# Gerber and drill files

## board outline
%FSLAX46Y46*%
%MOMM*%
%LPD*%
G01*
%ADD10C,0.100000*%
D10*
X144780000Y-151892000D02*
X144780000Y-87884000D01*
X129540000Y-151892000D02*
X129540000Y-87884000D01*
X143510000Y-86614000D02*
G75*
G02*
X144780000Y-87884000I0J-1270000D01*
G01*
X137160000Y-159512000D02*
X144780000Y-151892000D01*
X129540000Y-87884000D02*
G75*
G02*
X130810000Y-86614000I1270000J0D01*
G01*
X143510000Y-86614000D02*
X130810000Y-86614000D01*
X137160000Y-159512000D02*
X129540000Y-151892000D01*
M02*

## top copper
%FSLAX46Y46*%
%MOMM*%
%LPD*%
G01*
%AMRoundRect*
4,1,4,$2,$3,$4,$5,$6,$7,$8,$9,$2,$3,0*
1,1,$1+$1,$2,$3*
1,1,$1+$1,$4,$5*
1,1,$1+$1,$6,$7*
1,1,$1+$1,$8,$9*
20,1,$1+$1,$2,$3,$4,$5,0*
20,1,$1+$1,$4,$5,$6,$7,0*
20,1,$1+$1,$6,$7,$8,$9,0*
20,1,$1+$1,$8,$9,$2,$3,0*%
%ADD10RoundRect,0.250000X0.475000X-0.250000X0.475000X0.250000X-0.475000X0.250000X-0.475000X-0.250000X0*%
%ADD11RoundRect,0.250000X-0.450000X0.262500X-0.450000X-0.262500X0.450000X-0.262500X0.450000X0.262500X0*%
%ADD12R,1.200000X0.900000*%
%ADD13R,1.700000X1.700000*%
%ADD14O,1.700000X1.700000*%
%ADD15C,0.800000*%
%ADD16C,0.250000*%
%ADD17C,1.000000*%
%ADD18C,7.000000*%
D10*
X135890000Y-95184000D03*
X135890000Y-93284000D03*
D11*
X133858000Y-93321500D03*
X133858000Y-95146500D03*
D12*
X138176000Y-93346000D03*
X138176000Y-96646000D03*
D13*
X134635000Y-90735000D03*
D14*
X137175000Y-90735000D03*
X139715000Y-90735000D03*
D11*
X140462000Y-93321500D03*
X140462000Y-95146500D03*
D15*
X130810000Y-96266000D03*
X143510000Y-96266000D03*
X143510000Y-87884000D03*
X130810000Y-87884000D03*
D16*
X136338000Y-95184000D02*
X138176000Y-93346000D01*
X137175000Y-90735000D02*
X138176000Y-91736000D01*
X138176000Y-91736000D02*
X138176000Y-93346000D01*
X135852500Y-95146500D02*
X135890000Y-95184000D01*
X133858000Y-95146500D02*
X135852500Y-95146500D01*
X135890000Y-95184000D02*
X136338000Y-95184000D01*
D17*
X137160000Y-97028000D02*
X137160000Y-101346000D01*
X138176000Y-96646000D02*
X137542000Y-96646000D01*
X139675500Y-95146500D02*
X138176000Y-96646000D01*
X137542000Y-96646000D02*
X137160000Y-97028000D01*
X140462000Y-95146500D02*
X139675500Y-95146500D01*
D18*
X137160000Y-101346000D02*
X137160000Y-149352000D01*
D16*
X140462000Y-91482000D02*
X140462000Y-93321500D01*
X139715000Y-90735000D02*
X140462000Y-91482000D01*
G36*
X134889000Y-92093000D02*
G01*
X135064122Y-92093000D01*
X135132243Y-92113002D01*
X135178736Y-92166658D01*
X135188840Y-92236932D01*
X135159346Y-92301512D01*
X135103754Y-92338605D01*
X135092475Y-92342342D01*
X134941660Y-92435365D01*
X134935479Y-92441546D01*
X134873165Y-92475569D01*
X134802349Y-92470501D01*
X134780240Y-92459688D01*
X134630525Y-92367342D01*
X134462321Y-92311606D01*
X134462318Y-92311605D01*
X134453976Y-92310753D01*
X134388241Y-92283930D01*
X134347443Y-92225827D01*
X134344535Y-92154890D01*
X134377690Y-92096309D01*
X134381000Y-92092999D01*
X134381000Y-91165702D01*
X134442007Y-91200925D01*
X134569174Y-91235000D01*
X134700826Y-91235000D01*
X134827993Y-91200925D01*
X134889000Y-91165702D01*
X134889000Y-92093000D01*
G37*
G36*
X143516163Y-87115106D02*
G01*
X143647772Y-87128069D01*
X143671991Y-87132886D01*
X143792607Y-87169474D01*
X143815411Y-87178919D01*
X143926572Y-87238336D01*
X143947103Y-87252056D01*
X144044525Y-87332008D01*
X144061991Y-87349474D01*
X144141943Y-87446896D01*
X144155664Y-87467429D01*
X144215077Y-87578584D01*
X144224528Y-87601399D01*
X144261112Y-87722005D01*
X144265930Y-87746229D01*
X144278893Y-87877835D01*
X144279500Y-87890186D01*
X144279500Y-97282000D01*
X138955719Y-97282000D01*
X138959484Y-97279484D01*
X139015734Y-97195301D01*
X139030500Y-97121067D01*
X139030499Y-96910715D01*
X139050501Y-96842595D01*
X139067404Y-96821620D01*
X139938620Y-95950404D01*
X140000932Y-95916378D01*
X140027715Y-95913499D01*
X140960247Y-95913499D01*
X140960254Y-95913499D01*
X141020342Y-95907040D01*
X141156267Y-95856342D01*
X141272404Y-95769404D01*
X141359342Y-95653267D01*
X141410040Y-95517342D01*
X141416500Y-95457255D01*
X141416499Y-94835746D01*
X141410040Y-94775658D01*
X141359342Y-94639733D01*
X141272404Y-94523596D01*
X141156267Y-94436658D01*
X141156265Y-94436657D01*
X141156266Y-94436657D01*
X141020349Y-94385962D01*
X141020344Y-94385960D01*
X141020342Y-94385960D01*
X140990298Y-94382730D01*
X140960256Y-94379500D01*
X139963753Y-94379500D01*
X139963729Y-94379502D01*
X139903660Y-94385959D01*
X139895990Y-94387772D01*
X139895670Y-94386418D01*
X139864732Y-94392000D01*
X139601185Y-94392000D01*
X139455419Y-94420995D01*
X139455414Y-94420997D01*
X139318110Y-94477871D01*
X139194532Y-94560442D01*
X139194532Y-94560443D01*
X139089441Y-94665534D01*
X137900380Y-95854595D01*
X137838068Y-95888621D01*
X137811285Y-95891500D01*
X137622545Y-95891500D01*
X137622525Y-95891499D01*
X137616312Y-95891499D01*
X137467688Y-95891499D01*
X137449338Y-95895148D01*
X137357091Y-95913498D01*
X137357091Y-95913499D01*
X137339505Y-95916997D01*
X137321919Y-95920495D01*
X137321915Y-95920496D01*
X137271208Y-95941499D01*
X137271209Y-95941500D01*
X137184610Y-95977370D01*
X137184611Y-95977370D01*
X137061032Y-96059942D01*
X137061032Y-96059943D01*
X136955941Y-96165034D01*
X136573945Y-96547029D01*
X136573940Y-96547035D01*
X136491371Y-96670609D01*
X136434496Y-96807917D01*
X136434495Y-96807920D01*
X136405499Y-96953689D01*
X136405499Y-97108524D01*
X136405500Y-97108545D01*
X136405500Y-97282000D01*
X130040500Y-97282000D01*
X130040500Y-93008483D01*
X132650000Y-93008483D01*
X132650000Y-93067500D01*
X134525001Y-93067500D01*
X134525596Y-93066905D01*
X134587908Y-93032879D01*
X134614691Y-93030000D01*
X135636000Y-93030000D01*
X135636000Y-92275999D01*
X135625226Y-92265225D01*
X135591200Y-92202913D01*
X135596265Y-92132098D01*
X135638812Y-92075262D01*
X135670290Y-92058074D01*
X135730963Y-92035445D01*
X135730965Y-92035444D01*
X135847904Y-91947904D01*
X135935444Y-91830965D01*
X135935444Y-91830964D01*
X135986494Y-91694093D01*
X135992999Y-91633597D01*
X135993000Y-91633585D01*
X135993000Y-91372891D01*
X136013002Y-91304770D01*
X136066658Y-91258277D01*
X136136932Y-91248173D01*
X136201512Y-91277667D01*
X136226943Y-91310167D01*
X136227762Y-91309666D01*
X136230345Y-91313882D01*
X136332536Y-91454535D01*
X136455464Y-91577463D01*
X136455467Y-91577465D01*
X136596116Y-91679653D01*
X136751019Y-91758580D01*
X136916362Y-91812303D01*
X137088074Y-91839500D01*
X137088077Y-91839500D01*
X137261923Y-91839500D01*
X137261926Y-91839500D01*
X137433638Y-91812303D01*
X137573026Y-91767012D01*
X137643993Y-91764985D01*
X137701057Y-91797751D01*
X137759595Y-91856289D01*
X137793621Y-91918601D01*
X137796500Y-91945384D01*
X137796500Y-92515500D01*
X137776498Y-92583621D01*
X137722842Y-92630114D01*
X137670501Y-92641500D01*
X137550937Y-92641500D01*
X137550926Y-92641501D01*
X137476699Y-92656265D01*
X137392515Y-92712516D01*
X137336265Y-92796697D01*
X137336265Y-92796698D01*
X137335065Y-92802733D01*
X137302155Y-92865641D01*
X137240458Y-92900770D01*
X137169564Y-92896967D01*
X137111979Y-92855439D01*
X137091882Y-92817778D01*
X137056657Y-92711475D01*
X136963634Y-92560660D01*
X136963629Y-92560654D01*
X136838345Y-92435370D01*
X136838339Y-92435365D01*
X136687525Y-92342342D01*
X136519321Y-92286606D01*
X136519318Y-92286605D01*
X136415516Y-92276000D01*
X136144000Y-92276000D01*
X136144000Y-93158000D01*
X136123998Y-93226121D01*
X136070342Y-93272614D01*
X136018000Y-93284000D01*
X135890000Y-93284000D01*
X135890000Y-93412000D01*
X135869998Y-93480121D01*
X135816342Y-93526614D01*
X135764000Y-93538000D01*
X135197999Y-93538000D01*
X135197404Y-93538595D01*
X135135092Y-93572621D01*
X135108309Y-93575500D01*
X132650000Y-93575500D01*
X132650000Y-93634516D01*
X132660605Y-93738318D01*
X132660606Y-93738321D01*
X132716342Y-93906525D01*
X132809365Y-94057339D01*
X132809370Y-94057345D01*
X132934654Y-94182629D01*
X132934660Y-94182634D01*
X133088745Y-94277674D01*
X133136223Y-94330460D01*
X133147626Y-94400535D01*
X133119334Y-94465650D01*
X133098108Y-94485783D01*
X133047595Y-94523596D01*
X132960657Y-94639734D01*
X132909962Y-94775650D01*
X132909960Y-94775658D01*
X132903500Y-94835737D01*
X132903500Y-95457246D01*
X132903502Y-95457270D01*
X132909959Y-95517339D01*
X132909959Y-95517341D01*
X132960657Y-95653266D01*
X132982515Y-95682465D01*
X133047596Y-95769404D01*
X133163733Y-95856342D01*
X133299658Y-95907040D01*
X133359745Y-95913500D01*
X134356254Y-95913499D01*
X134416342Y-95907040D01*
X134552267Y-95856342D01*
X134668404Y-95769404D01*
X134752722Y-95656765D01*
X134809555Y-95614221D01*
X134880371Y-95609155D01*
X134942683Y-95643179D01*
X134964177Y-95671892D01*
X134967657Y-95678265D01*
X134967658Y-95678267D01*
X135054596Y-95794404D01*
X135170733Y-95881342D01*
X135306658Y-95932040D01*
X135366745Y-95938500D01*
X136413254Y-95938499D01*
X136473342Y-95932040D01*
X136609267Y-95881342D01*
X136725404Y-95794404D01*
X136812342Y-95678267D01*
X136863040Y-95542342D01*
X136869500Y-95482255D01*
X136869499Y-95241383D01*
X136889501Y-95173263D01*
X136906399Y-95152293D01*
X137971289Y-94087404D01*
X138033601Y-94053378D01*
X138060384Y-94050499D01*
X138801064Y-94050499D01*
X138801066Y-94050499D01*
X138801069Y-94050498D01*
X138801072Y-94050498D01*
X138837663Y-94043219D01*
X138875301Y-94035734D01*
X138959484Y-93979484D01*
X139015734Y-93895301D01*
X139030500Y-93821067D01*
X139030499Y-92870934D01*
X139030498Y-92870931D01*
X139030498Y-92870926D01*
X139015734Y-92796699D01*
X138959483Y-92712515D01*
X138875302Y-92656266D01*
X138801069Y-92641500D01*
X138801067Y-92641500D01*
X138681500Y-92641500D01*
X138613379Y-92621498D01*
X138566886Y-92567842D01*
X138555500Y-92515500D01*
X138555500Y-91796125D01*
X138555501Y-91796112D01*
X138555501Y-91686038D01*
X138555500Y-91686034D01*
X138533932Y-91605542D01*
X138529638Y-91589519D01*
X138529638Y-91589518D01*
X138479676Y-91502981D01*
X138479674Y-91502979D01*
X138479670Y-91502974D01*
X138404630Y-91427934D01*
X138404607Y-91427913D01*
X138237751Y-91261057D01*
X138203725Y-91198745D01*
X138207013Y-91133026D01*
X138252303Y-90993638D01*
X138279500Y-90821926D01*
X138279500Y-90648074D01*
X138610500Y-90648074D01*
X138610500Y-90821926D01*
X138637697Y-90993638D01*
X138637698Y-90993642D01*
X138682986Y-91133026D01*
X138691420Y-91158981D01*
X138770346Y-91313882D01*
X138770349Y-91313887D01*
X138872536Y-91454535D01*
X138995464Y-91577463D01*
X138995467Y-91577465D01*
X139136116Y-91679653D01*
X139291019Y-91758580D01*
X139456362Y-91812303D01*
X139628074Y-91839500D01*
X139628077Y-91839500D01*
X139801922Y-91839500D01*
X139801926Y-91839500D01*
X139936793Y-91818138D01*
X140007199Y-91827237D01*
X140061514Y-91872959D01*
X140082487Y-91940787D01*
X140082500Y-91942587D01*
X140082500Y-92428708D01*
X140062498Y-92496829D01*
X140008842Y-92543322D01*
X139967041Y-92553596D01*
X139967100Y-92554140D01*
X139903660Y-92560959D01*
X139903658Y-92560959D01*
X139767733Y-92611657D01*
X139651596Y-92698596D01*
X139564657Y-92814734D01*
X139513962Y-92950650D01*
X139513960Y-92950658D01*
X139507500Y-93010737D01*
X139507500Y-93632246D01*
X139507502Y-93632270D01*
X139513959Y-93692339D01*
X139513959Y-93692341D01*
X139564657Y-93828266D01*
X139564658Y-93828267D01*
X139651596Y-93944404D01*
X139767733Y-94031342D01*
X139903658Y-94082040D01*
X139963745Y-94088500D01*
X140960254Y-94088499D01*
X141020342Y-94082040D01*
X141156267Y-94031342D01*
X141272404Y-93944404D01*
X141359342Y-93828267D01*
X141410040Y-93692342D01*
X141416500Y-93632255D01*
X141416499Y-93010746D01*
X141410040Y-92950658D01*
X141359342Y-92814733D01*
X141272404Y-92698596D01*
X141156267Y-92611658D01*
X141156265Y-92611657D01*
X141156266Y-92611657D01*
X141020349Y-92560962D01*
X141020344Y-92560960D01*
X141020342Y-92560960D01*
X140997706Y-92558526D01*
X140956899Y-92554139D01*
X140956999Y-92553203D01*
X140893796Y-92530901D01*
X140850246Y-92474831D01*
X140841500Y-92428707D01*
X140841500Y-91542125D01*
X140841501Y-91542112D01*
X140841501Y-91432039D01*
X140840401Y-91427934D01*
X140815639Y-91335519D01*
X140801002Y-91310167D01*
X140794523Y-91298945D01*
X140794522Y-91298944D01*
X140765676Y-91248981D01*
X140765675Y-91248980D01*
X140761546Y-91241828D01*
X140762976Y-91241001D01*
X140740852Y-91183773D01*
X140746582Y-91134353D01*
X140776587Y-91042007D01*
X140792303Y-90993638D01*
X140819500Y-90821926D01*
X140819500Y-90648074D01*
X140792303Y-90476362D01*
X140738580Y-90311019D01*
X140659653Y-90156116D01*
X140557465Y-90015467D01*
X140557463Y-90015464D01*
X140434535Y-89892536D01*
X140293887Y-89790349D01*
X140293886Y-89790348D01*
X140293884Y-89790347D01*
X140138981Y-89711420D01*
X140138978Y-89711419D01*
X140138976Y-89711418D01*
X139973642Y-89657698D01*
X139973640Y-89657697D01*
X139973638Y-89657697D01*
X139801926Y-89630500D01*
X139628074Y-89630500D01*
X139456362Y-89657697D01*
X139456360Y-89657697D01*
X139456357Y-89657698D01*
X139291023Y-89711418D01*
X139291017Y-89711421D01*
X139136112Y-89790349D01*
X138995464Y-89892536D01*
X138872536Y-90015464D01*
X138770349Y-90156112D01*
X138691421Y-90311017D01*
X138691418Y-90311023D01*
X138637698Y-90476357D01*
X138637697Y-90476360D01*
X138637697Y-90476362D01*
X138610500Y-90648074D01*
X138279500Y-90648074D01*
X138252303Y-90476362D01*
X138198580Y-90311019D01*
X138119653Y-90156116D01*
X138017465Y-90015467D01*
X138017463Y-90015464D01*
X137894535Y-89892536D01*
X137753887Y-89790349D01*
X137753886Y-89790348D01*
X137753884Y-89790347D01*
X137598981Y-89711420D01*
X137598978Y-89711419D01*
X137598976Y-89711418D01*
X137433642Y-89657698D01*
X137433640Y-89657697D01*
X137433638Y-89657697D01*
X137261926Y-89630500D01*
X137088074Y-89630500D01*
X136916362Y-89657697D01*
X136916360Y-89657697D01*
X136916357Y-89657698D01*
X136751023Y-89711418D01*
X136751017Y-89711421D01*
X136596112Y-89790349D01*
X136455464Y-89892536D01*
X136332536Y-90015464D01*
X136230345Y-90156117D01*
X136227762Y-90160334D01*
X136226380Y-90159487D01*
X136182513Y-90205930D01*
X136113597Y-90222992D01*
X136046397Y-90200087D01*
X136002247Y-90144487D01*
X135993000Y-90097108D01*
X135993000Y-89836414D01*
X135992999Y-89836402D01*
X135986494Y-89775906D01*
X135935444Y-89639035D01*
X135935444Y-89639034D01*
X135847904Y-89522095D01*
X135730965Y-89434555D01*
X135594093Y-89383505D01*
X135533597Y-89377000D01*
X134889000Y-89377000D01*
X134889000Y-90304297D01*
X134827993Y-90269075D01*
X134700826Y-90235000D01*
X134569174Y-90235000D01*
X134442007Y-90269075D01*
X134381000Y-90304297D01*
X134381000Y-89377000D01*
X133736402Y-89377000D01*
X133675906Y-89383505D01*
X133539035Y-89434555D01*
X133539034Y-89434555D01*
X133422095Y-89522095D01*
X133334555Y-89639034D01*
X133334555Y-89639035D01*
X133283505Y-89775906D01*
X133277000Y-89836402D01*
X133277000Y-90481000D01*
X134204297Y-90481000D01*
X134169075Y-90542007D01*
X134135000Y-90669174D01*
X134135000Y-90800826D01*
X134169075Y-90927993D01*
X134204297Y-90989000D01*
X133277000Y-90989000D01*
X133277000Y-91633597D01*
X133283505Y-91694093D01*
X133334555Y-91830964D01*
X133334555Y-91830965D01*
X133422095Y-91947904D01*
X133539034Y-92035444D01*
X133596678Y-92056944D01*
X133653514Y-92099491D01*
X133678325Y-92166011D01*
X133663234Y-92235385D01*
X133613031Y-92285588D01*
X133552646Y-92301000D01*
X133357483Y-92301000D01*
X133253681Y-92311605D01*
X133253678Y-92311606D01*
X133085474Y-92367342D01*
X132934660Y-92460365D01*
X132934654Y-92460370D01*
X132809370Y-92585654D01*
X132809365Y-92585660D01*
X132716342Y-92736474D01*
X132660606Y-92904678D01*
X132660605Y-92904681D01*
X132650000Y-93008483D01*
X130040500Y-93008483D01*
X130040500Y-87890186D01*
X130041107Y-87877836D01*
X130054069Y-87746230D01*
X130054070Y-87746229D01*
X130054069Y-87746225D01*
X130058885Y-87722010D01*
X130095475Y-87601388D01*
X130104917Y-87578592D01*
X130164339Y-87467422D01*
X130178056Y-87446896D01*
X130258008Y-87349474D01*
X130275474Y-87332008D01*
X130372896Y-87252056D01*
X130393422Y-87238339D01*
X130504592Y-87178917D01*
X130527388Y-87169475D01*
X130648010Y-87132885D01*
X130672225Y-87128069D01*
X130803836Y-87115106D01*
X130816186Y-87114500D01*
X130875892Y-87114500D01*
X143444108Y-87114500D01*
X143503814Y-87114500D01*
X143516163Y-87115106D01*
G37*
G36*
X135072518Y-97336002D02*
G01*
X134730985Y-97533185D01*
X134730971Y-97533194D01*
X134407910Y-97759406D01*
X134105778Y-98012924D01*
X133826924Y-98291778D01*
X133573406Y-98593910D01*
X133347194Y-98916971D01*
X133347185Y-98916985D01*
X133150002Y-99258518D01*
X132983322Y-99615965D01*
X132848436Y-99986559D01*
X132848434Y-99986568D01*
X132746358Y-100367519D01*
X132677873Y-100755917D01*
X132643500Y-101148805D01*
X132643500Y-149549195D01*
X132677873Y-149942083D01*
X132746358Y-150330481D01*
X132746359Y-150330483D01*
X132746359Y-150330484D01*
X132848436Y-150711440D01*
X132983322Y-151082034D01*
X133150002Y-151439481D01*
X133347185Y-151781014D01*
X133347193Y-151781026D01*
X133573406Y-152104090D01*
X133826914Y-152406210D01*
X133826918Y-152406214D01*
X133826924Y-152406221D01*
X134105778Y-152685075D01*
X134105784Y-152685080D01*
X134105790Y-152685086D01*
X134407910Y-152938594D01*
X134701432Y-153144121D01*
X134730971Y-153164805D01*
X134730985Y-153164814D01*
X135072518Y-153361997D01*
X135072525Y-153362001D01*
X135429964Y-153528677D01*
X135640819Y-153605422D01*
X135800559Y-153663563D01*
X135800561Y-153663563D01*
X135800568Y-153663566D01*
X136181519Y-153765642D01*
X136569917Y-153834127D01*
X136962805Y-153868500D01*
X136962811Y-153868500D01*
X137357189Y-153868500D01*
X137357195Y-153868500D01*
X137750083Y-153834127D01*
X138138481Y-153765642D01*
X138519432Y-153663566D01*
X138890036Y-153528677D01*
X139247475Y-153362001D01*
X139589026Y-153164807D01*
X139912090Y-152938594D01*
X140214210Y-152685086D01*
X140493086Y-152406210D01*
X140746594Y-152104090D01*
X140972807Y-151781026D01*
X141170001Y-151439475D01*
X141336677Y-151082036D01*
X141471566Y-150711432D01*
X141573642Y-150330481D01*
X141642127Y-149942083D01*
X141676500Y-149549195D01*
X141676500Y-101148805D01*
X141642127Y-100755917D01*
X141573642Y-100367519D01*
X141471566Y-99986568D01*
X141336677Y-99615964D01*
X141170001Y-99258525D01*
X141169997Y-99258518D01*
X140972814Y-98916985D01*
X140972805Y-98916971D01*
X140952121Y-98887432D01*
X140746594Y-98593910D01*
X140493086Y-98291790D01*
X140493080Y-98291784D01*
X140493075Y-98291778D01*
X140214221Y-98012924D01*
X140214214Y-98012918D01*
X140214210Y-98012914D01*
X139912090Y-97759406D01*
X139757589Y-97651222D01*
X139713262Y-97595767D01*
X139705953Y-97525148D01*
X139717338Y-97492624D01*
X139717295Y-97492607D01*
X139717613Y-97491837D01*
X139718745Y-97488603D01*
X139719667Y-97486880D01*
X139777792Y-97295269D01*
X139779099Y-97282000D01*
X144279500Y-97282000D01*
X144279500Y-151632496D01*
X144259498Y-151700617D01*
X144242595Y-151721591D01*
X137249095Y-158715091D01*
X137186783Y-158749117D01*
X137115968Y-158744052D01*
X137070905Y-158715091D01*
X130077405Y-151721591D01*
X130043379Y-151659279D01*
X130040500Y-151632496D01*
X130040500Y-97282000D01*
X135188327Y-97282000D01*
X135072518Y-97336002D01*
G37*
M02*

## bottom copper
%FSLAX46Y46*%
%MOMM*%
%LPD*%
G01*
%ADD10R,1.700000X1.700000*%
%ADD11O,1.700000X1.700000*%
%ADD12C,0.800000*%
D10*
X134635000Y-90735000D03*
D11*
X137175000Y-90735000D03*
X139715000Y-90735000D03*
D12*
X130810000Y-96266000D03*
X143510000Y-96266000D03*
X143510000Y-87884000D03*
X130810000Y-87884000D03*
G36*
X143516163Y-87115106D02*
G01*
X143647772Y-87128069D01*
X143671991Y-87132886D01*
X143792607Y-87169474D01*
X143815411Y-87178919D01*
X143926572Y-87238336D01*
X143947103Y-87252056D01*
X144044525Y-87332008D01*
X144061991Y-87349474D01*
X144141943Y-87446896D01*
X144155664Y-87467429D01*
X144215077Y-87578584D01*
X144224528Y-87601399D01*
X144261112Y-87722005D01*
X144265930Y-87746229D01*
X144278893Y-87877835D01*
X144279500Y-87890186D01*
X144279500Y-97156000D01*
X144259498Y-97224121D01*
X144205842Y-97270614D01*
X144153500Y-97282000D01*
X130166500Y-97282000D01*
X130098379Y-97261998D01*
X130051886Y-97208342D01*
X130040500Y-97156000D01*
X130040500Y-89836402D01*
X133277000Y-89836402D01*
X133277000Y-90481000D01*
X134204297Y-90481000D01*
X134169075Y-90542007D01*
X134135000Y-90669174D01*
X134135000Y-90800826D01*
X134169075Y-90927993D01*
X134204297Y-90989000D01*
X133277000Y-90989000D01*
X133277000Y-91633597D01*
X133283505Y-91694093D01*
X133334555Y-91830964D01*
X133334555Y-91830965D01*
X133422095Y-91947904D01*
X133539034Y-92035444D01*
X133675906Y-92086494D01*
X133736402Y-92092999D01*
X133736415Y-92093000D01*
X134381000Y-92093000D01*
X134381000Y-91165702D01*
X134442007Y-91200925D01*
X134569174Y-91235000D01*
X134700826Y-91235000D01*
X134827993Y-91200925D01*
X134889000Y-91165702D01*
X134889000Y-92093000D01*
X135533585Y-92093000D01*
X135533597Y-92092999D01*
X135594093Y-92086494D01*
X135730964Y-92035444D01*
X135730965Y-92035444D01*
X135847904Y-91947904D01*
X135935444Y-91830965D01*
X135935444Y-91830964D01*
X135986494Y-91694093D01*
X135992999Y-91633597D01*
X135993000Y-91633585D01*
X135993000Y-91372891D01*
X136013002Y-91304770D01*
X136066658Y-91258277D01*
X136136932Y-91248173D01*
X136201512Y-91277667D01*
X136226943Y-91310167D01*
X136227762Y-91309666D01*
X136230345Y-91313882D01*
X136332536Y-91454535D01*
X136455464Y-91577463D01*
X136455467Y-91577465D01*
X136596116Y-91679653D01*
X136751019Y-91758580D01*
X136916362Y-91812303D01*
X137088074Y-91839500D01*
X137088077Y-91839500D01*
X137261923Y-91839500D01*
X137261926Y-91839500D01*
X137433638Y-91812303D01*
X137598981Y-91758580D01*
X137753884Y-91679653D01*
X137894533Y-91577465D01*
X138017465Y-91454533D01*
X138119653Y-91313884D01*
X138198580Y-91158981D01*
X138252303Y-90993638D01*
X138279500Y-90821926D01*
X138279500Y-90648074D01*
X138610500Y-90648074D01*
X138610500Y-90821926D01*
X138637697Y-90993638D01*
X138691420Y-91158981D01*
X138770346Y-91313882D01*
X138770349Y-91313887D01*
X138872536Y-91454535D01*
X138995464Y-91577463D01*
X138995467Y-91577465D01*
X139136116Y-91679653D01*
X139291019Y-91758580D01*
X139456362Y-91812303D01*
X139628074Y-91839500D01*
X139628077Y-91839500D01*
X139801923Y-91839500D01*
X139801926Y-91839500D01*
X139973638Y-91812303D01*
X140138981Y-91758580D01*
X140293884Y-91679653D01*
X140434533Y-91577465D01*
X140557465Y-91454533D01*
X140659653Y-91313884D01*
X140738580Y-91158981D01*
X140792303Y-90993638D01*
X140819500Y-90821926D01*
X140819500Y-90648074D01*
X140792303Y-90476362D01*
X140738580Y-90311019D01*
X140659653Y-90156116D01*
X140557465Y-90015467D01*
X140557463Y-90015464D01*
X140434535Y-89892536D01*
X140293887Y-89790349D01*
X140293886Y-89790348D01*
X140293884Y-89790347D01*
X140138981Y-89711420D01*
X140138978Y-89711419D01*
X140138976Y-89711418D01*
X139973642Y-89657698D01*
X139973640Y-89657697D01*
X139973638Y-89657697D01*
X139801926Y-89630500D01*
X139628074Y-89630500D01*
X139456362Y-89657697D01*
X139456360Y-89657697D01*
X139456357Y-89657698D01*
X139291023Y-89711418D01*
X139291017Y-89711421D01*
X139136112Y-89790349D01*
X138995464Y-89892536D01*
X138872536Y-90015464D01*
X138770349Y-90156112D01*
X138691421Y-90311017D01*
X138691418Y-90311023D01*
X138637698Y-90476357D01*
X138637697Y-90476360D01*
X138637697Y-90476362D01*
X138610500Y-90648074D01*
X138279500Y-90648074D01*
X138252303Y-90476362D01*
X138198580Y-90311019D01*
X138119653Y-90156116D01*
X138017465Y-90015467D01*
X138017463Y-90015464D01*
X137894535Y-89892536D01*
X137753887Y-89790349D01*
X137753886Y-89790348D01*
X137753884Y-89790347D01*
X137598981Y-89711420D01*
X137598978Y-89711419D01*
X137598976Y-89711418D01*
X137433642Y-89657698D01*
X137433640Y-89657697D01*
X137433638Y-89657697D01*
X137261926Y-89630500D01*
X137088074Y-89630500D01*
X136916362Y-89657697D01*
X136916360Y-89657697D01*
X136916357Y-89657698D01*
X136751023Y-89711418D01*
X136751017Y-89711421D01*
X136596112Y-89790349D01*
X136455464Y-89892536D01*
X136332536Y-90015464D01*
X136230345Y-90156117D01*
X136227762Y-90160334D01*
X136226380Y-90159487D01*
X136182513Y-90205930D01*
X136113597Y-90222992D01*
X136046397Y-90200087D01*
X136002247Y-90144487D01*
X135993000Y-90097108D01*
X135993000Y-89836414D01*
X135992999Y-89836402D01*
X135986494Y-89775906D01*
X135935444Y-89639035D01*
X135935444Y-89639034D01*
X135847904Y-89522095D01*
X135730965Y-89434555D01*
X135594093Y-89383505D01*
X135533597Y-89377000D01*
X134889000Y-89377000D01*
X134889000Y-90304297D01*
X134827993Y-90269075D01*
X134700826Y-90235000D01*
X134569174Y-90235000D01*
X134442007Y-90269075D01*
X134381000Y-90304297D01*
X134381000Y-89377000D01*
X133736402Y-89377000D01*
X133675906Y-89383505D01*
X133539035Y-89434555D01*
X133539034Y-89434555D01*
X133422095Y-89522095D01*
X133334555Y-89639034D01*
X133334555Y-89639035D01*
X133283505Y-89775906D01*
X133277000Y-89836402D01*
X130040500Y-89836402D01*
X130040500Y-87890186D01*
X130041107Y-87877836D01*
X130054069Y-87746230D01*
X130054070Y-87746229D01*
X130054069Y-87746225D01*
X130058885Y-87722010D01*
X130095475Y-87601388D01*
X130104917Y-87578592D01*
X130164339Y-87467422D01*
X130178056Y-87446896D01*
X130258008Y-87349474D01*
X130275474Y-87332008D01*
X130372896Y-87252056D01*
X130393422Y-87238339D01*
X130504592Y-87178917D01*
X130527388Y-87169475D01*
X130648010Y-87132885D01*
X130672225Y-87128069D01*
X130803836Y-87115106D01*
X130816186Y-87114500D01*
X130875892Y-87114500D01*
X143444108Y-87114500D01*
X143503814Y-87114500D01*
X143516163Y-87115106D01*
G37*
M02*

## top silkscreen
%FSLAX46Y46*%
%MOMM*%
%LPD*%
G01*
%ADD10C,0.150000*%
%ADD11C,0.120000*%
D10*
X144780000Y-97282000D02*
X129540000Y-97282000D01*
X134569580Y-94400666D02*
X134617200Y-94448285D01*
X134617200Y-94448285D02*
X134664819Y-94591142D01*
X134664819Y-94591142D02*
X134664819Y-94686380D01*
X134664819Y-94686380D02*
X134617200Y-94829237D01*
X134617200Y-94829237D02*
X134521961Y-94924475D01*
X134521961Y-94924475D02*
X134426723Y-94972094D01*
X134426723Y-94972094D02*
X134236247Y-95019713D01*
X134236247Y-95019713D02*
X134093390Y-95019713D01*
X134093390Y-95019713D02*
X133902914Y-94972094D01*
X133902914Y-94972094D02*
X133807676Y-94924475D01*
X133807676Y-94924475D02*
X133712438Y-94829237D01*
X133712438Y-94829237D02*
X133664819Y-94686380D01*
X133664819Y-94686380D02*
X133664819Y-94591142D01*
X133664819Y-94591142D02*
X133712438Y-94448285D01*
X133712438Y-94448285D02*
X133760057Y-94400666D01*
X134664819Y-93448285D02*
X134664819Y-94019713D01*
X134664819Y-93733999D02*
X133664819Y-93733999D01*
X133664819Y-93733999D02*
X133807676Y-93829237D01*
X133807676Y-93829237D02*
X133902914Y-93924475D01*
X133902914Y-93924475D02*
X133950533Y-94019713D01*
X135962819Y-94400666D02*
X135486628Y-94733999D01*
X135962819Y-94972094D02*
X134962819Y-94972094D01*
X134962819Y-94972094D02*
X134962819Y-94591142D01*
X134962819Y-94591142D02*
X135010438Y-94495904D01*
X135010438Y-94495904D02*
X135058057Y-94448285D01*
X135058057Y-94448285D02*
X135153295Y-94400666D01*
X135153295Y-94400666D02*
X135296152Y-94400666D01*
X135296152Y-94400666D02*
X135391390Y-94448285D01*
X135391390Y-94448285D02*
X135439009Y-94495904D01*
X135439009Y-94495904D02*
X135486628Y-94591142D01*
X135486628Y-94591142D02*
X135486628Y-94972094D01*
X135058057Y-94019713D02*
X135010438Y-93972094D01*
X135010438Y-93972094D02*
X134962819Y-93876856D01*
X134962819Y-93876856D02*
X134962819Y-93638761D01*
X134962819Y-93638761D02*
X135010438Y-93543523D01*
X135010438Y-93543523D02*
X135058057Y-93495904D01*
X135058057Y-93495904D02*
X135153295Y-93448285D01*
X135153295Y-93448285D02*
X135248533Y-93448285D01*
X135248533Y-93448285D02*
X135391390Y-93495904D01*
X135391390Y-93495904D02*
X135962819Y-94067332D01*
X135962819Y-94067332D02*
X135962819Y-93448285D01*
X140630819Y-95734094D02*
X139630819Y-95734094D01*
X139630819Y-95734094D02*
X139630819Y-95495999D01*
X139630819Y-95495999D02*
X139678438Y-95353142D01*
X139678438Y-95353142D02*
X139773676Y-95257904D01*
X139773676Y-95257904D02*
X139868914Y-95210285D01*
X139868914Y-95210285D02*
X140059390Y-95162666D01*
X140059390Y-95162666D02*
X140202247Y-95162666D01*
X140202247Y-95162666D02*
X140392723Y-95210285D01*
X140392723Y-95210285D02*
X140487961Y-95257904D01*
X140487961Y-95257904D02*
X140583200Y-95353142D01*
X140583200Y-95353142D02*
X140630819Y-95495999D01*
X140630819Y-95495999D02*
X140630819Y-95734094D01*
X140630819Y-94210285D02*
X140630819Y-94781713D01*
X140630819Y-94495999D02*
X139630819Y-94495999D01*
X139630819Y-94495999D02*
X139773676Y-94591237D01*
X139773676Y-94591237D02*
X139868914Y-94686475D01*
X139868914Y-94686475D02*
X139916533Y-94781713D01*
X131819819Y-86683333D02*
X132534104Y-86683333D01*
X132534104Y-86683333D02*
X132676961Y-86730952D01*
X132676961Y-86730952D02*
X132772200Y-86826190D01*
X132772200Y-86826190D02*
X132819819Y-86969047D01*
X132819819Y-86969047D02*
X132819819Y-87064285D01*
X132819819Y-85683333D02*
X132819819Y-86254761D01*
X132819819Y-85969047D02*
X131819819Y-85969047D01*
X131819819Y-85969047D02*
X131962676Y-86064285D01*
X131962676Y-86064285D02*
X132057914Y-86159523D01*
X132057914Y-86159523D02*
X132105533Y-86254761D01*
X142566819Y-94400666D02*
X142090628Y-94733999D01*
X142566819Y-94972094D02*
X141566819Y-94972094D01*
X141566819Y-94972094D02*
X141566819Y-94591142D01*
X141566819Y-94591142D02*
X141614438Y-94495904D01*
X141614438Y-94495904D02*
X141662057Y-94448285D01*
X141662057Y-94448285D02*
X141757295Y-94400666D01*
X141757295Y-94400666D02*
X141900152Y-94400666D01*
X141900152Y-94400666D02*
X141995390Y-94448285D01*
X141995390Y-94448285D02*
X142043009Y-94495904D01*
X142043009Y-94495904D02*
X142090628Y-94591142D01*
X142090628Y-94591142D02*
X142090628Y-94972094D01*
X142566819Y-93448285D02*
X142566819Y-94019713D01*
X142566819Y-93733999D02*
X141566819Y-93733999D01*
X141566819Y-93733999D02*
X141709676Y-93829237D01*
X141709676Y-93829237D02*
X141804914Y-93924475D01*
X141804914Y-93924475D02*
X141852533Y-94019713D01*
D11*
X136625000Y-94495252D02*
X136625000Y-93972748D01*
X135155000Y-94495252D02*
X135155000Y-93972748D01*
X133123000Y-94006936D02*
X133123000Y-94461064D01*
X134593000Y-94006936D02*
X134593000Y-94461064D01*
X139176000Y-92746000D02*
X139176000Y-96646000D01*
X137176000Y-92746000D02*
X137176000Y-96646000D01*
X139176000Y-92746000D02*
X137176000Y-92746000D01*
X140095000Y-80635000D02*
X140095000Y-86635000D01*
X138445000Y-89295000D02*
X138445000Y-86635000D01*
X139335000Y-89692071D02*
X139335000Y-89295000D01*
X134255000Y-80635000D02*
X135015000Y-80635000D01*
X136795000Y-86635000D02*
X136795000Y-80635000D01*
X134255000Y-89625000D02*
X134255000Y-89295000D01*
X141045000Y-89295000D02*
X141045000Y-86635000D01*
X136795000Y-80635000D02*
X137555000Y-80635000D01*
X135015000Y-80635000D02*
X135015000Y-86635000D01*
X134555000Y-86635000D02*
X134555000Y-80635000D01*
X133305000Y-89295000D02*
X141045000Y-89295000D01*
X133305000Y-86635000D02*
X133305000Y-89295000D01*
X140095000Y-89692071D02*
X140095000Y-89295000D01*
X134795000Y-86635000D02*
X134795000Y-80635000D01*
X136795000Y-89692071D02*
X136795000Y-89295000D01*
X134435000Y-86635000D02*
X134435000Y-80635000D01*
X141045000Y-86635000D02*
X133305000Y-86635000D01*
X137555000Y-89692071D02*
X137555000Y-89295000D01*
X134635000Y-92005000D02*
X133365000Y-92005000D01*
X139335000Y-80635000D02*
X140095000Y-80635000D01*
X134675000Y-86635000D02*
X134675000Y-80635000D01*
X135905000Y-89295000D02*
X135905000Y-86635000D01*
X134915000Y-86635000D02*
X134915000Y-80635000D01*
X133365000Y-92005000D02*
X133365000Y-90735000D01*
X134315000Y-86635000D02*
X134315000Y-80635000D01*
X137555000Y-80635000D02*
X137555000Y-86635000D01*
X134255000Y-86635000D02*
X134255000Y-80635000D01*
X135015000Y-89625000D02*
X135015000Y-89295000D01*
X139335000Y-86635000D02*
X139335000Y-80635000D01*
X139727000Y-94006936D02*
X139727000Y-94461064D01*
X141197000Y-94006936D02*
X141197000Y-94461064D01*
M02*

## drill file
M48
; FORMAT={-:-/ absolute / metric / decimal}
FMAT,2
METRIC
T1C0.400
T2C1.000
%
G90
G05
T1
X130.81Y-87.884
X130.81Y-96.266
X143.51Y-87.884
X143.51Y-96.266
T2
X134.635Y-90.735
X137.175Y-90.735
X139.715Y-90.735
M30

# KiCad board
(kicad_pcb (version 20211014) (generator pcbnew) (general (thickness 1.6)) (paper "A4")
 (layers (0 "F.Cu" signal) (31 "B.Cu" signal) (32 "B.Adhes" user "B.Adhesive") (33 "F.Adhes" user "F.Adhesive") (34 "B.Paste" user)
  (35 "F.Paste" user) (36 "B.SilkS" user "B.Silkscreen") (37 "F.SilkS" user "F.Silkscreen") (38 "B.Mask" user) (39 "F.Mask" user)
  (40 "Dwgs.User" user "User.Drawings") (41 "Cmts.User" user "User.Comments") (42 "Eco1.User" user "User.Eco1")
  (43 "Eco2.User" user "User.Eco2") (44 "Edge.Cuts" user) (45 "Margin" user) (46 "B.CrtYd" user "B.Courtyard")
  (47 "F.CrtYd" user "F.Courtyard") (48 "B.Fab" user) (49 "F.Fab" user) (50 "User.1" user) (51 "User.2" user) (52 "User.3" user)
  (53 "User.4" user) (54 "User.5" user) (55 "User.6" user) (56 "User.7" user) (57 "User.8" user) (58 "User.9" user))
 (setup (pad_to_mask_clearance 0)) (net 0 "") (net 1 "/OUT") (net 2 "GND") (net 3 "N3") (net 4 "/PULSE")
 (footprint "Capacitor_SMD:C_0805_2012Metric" (layer "F.Cu") (at 135.89 94.234 90)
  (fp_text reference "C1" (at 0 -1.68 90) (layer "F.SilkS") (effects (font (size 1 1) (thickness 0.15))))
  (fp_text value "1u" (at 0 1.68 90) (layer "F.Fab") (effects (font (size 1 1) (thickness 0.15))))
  (fp_line (start -0.261252 0.735) (end 0.261252 0.735) (layer "F.SilkS") (width 0.12))
  (fp_line (start -0.261252 -0.735) (end 0.261252 -0.735) (layer "F.SilkS") (width 0.12))
  (pad "1" smd roundrect (at -0.95 0 90) (size 1 1.45) (layers "F.Cu" "F.Paste" "F.Mask") (roundrect_rratio 0.25) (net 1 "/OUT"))
  (pad "2" smd roundrect (at 0.95 0 90) (size 1 1.45) (layers "F.Cu" "F.Paste" "F.Mask") (roundrect_rratio 0.25) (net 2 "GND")))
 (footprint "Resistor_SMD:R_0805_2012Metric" (layer "F.Cu") (at 133.858 94.234 -90)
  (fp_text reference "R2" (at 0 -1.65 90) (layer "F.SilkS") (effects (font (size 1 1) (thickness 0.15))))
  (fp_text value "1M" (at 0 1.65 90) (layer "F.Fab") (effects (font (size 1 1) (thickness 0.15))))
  (fp_line (start -0.227064 0.735) (end 0.227064 0.735) (layer "F.SilkS") (width 0.12))
  (fp_line (start -0.227064 -0.735) (end 0.227064 -0.735) (layer "F.SilkS") (width 0.12))
  (pad "1" smd roundrect (at -0.9125 0 270) (size 1.025 1.4) (layers "F.Cu" "F.Paste" "F.Mask") (roundrect_rratio 0.243902) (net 2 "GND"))
  (pad "2" smd roundrect (at 0.9125 0 270) (size 1.025 1.4) (layers "F.Cu" "F.Paste" "F.Mask") (roundrect_rratio 0.243902) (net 1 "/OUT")))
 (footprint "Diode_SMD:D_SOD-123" (layer "F.Cu") (at 138.176 94.996 -90)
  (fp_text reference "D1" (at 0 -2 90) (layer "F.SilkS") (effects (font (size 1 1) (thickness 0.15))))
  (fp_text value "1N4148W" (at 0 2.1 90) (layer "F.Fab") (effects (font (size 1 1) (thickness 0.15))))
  (fp_line (start -2.25 -1) (end 1.65 -1) (layer "F.SilkS") (width 0.12))
  (fp_line (start -2.25 1) (end 1.65 1) (layer "F.SilkS") (width 0.12))
  (fp_line (start -2.25 -1) (end -2.25 1) (layer "F.SilkS") (width 0.12))
  (pad "1" smd rect (at -1.65 0 270) (size 0.9 1.2) (layers "F.Cu" "F.Paste" "F.Mask") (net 1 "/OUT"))
  (pad "2" smd rect (at 1.65 0 270) (size 0.9 1.2) (layers "F.Cu" "F.Paste" "F.Mask") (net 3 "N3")))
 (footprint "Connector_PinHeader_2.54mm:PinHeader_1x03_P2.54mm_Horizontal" (layer "F.Cu") (at 134.635 90.735 90)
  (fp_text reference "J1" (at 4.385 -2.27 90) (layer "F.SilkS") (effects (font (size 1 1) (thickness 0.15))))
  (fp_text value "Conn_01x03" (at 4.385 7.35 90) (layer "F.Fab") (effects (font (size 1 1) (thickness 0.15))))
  (fp_line (start 10.1 5.46) (end 4.1 5.46) (layer "F.SilkS") (width 0.12))
  (fp_line (start 1.44 3.81) (end 4.1 3.81) (layer "F.SilkS") (width 0.12))
  (fp_line (start 1.042929 4.7) (end 1.44 4.7) (layer "F.SilkS") (width 0.12))
  (fp_line (start 10.1 -0.38) (end 10.1 0.38) (layer "F.SilkS") (width 0.12))
  (fp_line (start 4.1 2.16) (end 10.1 2.16) (layer "F.SilkS") (width 0.12))
  (fp_line (start 1.11 -0.38) (end 1.44 -0.38) (layer "F.SilkS") (width 0.12))
  (fp_line (start 1.44 6.41) (end 4.1 6.41) (layer "F.SilkS") (width 0.12))
  (fp_line (start 10.1 2.16) (end 10.1 2.92) (layer "F.SilkS") (width 0.12))
  (fp_line (start 10.1 0.38) (end 4.1 0.38) (layer "F.SilkS") (width 0.12))
  (fp_line (start 4.1 -0.08) (end 10.1 -0.08) (layer "F.SilkS") (width 0.12))
  (fp_line (start 1.44 -1.33) (end 1.44 6.41) (layer "F.SilkS") (width 0.12))
  (fp_line (start 4.1 -1.33) (end 1.44 -1.33) (layer "F.SilkS") (width 0.12))
  (fp_line (start 1.042929 5.46) (end 1.44 5.46) (layer "F.SilkS") (width 0.12))
  (fp_line (start 4.1 0.16) (end 10.1 0.16) (layer "F.SilkS") (width 0.12))
  (fp_line (start 1.042929 2.16) (end 1.44 2.16) (layer "F.SilkS") (width 0.12))
  (fp_line (start 4.1 -0.2) (end 10.1 -0.2) (layer "F.SilkS") (width 0.12))
  (fp_line (start 4.1 6.41) (end 4.1 -1.33) (layer "F.SilkS") (width 0.12))
  (fp_line (start 1.042929 2.92) (end 1.44 2.92) (layer "F.SilkS") (width 0.12))
  (fp_line (start -1.27 0) (end -1.27 -1.27) (layer "F.SilkS") (width 0.12))
  (fp_line (start 10.1 4.7) (end 10.1 5.46) (layer "F.SilkS") (width 0.12))
  (fp_line (start 4.1 0.04) (end 10.1 0.04) (layer "F.SilkS") (width 0.12))
  (fp_line (start 1.44 1.27) (end 4.1 1.27) (layer "F.SilkS") (width 0.12))
  (fp_line (start 4.1 0.28) (end 10.1 0.28) (layer "F.SilkS") (width 0.12))
  (fp_line (start -1.27 -1.27) (end 0 -1.27) (layer "F.SilkS") (width 0.12))
  (fp_line (start 4.1 -0.32) (end 10.1 -0.32) (layer "F.SilkS") (width 0.12))
  (fp_line (start 10.1 2.92) (end 4.1 2.92) (layer "F.SilkS") (width 0.12))
  (fp_line (start 4.1 -0.38) (end 10.1 -0.38) (layer "F.SilkS") (width 0.12))
  (fp_line (start 1.11 0.38) (end 1.44 0.38) (layer "F.SilkS") (width 0.12))
  (fp_line (start 4.1 4.7) (end 10.1 4.7) (layer "F.SilkS") (width 0.12))
  (pad "1" thru_hole rect (at 0 0 90) (size 1.7 1.7) (drill 1) (layers *.Cu *.Mask) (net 2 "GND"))
  (pad "2" thru_hole oval (at 0 2.54 90) (size 1.7 1.7) (drill 1) (layers *.Cu *.Mask) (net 1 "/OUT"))
  (pad "3" thru_hole oval (at 0 5.08 90) (size 1.7 1.7) (drill 1) (layers *.Cu *.Mask) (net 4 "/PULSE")))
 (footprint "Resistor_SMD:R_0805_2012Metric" (layer "F.Cu") (at 140.462 94.234 -90)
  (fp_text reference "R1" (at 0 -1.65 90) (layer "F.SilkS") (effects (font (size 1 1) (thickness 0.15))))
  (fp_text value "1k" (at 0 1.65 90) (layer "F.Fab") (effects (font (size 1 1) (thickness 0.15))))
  (fp_line (start -0.227064 0.735) (end 0.227064 0.735) (layer "F.SilkS") (width 0.12))
  (fp_line (start -0.227064 -0.735) (end 0.227064 -0.735) (layer "F.SilkS") (width 0.12))
  (pad "1" smd roundrect (at -0.9125 0 270) (size 1.025 1.4) (layers "F.Cu" "F.Paste" "F.Mask") (roundrect_rratio 0.243902) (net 4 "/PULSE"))
  (pad "2" smd roundrect (at 0.9125 0 270) (size 1.025 1.4) (layers "F.Cu" "F.Paste" "F.Mask") (roundrect_rratio 0.243902) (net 3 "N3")))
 (gr_line (start 144.78 97.282) (end 129.54 97.282) (layer "F.SilkS") (width 0.15))
 (gr_line (start 144.78 151.892) (end 144.78 87.884) (layer "Edge.Cuts") (width 0.1))
 (gr_line (start 129.54 151.892) (end 129.54 87.884) (layer "Edge.Cuts") (width 0.1))
 (gr_arc (start 143.51 86.614) (mid 144.408026 86.985974) (end 144.78 87.884) (layer "Edge.Cuts") (width 0.1))
 (gr_line (start 137.16 159.512) (end 144.78 151.892) (layer "Edge.Cuts") (width 0.1))
 (gr_arc (start 129.54 87.884) (mid 129.911974 86.985974) (end 130.81 86.614) (layer "Edge.Cuts") (width 0.1))
 (gr_line (start 143.51 86.614) (end 130.81 86.614) (layer "Edge.Cuts") (width 0.1))
 (gr_line (start 137.16 159.512) (end 129.54 151.892) (layer "Edge.Cuts") (width 0.1))
 (segment (start 136.338 95.184) (end 138.176 93.346) (width 0.25) (layer "F.Cu") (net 1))
 (segment (start 137.175 90.735) (end 138.176 91.736) (width 0.25) (layer "F.Cu") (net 1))
 (segment (start 138.176 91.736) (end 138.176 93.346) (width 0.25) (layer "F.Cu") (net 1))
 (segment (start 135.8525 95.1465) (end 135.89 95.184) (width 0.25) (layer "F.Cu") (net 1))
 (segment (start 133.858 95.1465) (end 135.8525 95.1465) (width 0.25) (layer "F.Cu") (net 1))
 (segment (start 135.89 95.184) (end 136.338 95.184) (width 0.25) (layer "F.Cu") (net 1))
 (via (at 130.81 96.266) (size 0.8) (drill 0.4) (layers "F.Cu" "B.Cu") (free) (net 2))
 (via (at 143.51 96.266) (size 0.8) (drill 0.4) (layers "F.Cu" "B.Cu") (free) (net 2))
 (via (at 143.51 87.884) (size 0.8) (drill 0.4) (layers "F.Cu" "B.Cu") (free) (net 2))
 (via (at 130.81 87.884) (size 0.8) (drill 0.4) (layers "F.Cu" "B.Cu") (free) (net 2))
 (segment (start 137.16 97.028) (end 137.16 101.346) (width 1) (layer "F.Cu") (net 3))
 (segment (start 138.176 96.646) (end 137.542 96.646) (width 1) (layer "F.Cu") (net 3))
 (segment (start 139.6755 95.1465) (end 138.176 96.646) (width 1) (layer "F.Cu") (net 3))
 (segment (start 137.542 96.646) (end 137.16 97.028) (width 1) (layer "F.Cu") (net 3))
 (segment (start 140.462 95.1465) (end 139.6755 95.1465) (width 1) (layer "F.Cu") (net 3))
 (segment (start 137.16 101.346) (end 137.16 149.352) (width 7) (layer "F.Cu") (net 3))
 (segment (start 140.462 91.482) (end 140.462 93.3215) (width 0.25) (layer "F.Cu") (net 4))
 (segment (start 139.715 90.735) (end 140.462 91.482) (width 0.25) (layer "F.Cu") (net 4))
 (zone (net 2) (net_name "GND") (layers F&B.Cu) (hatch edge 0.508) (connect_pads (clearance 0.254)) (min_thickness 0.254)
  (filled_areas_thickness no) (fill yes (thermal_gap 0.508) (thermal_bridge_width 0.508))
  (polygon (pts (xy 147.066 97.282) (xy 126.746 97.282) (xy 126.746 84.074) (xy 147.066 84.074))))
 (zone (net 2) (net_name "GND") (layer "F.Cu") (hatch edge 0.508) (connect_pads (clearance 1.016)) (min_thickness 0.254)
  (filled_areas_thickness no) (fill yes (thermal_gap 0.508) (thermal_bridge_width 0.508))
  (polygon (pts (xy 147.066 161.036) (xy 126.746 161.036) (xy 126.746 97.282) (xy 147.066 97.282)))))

